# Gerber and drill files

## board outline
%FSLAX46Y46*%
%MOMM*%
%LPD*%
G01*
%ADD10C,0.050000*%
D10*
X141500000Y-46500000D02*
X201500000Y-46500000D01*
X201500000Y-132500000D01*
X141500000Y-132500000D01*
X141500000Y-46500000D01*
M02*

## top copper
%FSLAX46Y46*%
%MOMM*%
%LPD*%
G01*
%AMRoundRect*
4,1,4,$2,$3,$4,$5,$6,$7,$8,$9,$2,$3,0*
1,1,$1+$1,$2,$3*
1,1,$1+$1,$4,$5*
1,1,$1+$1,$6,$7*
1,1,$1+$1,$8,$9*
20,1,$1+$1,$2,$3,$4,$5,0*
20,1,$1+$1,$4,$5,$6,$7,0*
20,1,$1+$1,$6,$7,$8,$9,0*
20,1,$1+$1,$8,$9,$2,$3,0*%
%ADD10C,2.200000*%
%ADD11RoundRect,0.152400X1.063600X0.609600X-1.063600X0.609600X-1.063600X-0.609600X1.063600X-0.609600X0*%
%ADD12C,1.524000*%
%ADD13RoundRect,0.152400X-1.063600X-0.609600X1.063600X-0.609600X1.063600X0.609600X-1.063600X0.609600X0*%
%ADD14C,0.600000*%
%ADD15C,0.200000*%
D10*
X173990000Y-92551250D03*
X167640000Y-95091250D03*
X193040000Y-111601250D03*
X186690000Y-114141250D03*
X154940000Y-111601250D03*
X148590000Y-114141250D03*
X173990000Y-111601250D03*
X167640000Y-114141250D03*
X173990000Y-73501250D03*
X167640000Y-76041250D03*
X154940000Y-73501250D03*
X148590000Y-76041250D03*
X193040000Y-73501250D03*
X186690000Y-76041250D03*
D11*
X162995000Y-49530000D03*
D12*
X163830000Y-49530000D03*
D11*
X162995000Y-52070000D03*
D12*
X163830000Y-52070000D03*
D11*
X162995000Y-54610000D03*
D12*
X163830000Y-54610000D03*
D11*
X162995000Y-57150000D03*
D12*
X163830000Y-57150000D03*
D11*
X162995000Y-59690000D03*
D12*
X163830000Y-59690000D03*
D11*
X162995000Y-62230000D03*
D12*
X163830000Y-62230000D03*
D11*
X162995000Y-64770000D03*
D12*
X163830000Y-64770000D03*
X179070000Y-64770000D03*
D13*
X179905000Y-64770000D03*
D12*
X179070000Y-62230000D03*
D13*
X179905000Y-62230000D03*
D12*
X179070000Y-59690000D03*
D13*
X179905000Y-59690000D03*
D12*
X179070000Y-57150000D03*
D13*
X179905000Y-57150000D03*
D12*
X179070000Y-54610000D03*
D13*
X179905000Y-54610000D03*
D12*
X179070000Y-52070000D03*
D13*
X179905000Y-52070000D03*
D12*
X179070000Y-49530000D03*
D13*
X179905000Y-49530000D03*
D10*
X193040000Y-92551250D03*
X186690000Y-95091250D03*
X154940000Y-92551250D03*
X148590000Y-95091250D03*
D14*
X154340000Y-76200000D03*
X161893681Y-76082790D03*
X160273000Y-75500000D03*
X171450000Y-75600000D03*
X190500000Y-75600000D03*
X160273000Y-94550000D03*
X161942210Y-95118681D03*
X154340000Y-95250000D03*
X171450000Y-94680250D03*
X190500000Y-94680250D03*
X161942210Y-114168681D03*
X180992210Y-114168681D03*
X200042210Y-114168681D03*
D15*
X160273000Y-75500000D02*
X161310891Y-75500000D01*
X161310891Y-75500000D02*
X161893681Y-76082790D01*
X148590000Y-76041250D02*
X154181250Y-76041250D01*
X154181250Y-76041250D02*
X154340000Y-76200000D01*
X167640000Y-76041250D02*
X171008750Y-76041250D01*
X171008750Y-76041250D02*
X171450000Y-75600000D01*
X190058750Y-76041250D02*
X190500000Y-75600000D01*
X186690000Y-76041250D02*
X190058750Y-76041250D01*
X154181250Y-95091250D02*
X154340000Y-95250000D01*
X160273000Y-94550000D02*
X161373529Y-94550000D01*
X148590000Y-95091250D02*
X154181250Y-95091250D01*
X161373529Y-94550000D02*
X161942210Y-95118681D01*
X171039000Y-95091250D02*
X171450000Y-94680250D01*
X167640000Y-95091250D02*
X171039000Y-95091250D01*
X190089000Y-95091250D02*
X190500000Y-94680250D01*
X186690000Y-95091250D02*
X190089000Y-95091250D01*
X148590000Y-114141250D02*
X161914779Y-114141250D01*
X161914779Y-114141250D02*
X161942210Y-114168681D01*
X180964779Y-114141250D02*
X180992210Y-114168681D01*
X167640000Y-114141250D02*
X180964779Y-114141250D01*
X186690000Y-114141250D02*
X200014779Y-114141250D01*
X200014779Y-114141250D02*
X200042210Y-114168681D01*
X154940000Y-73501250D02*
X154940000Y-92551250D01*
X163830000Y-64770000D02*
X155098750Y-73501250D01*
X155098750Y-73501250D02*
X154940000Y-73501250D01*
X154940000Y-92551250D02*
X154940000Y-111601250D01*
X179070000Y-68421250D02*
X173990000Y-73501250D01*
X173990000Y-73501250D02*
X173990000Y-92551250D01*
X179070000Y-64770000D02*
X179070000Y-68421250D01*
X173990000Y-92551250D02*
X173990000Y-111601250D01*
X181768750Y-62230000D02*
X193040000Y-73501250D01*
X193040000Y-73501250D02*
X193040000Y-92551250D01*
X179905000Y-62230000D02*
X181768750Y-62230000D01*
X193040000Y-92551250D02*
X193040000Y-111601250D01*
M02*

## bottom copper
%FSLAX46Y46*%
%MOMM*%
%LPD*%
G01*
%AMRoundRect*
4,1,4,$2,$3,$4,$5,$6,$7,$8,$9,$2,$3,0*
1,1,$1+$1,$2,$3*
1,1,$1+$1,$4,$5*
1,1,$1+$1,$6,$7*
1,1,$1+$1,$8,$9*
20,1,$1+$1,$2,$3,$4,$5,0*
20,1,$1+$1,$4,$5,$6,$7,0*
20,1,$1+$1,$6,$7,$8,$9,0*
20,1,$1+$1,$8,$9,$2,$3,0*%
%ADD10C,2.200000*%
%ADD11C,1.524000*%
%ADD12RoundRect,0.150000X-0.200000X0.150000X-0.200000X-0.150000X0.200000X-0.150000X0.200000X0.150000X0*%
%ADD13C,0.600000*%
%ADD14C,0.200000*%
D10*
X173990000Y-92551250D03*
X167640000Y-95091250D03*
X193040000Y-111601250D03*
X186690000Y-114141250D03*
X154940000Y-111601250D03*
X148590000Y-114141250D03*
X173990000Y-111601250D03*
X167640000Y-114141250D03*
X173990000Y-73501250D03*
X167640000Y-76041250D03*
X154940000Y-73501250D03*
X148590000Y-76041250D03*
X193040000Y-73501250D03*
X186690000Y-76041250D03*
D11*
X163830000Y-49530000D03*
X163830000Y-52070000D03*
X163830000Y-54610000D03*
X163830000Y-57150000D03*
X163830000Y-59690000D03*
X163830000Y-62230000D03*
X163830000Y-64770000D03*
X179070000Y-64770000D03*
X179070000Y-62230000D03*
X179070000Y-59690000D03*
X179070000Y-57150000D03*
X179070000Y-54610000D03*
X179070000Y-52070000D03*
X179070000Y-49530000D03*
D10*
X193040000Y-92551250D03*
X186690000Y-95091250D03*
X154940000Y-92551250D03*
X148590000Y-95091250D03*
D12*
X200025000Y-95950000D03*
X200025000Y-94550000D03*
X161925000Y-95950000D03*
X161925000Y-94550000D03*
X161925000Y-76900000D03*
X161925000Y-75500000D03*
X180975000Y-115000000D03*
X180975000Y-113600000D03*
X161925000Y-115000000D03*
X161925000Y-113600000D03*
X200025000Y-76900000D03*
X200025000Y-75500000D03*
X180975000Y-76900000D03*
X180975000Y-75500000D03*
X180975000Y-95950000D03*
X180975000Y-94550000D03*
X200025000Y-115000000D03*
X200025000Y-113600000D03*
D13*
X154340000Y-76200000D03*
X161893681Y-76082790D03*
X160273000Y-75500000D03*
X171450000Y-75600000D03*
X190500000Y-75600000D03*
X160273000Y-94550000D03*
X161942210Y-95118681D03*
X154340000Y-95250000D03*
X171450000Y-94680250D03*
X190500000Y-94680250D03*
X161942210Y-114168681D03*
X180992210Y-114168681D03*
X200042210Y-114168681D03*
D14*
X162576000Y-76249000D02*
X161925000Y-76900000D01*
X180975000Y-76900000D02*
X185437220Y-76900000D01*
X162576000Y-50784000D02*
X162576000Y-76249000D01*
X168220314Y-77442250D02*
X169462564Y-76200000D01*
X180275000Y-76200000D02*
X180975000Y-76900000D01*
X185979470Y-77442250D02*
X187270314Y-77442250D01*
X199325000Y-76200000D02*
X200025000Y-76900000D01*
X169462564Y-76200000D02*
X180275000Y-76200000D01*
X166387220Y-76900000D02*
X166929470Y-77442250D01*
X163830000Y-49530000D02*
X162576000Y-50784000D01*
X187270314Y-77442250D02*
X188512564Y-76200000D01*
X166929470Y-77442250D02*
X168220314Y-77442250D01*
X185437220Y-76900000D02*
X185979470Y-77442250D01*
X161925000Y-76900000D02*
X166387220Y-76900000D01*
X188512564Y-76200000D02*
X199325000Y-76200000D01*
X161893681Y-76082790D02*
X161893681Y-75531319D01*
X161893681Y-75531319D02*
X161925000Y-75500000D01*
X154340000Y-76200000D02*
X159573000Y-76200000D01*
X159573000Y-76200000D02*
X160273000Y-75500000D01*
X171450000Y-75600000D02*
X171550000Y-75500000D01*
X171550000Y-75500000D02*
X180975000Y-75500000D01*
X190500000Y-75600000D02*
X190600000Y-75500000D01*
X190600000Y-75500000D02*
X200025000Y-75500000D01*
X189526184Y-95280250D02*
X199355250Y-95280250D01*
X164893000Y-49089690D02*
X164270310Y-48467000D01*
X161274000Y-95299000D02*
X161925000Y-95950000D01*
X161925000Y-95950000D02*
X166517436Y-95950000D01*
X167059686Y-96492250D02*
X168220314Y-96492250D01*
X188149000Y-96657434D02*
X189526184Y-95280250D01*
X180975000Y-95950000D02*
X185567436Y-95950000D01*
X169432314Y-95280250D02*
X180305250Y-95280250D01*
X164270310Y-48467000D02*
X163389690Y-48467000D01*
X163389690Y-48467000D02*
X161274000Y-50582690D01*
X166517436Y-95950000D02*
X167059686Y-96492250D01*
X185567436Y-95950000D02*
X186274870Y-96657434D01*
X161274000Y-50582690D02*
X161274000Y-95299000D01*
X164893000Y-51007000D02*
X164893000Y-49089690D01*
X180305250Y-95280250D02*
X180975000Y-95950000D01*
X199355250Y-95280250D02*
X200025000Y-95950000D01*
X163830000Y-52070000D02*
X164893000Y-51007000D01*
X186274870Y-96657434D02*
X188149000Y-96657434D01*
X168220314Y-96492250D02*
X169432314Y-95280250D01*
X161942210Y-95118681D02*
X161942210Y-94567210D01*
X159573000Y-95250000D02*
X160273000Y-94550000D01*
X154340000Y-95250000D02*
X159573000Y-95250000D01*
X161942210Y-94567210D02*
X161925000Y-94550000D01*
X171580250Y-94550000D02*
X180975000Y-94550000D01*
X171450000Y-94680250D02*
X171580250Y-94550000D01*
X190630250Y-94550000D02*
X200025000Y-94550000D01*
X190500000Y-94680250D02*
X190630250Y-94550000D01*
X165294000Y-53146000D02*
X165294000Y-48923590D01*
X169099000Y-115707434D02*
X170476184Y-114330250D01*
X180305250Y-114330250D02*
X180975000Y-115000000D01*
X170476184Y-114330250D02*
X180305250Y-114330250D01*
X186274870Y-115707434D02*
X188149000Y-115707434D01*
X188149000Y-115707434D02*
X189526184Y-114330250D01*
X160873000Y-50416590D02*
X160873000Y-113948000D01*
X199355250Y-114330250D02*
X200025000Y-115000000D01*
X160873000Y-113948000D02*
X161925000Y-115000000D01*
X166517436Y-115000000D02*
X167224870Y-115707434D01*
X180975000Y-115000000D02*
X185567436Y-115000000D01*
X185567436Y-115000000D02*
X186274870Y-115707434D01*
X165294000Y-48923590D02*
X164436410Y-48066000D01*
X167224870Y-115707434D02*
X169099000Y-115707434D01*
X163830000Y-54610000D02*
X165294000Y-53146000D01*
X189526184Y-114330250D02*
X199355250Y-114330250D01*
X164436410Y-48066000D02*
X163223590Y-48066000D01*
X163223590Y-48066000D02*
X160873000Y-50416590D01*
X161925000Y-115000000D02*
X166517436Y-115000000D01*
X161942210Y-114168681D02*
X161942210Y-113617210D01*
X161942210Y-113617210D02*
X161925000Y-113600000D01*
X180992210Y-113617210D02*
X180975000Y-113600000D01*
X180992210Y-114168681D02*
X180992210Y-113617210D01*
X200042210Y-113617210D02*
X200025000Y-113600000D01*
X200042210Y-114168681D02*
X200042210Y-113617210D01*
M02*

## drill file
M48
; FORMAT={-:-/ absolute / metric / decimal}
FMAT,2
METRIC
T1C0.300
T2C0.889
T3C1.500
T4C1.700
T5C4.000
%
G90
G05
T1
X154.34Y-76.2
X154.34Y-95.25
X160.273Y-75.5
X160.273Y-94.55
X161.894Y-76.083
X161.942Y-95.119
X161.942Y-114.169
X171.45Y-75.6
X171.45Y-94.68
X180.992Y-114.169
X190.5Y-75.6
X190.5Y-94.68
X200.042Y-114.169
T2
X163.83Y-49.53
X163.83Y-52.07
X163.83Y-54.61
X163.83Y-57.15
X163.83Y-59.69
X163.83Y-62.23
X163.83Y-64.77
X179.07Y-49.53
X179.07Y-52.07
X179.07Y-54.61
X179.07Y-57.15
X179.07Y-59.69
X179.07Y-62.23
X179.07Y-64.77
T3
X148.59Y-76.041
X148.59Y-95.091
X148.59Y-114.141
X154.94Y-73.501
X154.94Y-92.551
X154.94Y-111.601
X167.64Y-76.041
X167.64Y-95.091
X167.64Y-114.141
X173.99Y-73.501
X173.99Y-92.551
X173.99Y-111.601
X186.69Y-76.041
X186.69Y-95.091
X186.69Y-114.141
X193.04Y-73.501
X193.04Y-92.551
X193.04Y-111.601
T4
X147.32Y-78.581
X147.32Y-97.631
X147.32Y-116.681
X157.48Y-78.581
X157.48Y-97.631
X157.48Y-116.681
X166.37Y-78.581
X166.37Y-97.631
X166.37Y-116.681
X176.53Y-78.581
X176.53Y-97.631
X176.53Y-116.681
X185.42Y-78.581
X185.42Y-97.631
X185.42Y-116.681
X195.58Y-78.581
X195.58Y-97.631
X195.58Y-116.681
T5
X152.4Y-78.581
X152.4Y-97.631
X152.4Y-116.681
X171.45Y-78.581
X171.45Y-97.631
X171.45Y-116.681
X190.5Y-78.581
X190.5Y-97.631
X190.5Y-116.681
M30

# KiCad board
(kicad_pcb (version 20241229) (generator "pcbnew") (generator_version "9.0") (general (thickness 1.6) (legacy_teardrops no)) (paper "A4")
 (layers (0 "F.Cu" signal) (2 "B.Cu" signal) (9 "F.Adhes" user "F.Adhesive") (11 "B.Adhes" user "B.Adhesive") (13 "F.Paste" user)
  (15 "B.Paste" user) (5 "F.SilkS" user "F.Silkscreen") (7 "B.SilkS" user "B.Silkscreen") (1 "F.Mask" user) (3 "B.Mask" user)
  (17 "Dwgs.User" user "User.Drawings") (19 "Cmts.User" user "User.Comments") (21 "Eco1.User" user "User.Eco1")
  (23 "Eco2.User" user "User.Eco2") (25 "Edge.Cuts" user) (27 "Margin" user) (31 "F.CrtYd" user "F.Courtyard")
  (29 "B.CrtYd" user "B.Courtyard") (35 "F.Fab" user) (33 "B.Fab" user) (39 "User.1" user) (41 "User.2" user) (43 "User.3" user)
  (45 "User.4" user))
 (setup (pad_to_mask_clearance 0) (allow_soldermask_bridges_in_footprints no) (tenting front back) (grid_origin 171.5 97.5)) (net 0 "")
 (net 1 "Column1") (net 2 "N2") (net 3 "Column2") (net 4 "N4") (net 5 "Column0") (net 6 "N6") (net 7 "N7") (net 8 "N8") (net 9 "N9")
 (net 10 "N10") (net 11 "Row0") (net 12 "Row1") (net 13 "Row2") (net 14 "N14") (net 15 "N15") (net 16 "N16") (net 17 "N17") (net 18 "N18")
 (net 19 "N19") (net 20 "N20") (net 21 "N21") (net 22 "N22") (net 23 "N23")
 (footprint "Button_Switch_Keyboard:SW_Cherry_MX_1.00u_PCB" (layer "F.Cu") (at 173.99 92.55125)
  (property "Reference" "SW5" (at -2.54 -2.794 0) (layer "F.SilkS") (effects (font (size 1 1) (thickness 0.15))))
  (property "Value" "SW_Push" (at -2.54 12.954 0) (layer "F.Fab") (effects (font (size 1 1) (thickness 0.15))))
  (pad "" np_thru_hole circle (at -7.62 5.08) (size 1.7 1.7) (drill 1.7) (layers "*.Cu" "*.Mask"))
  (pad "" np_thru_hole circle (at -2.54 5.08) (size 4 4) (drill 4) (layers "*.Cu" "*.Mask"))
  (pad "" np_thru_hole circle (at 2.54 5.08) (size 1.7 1.7) (drill 1.7) (layers "*.Cu" "*.Mask"))
  (pad "1" thru_hole circle (at 0 0) (size 2.2 2.2) (drill 1.5) (layers "*.Cu" "*.Mask") (remove_unused_layers no) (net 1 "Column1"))
  (pad "2" thru_hole circle (at -6.35 2.54) (size 2.2 2.2) (drill 1.5) (layers "*.Cu" "*.Mask") (remove_unused_layers no) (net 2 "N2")))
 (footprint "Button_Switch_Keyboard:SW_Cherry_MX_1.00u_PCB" (layer "F.Cu") (at 193.04 111.60125)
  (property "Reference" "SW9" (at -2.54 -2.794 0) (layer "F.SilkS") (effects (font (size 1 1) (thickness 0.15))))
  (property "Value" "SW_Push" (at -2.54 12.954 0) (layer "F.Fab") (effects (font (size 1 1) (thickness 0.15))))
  (pad "" np_thru_hole circle (at -7.62 5.08) (size 1.7 1.7) (drill 1.7) (layers "*.Cu" "*.Mask"))
  (pad "" np_thru_hole circle (at -2.54 5.08) (size 4 4) (drill 4) (layers "*.Cu" "*.Mask"))
  (pad "" np_thru_hole circle (at 2.54 5.08) (size 1.7 1.7) (drill 1.7) (layers "*.Cu" "*.Mask"))
  (pad "1" thru_hole circle (at 0 0) (size 2.2 2.2) (drill 1.5) (layers "*.Cu" "*.Mask") (remove_unused_layers no) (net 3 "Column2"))
  (pad "2" thru_hole circle (at -6.35 2.54) (size 2.2 2.2) (drill 1.5) (layers "*.Cu" "*.Mask") (remove_unused_layers no) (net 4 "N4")))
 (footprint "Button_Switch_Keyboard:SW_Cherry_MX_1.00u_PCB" (layer "F.Cu") (at 154.94 111.60125)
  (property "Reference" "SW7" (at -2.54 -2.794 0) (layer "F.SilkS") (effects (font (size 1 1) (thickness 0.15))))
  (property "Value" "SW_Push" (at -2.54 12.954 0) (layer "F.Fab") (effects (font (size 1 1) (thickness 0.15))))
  (pad "" np_thru_hole circle (at -7.62 5.08) (size 1.7 1.7) (drill 1.7) (layers "*.Cu" "*.Mask"))
  (pad "" np_thru_hole circle (at -2.54 5.08) (size 4 4) (drill 4) (layers "*.Cu" "*.Mask"))
  (pad "" np_thru_hole circle (at 2.54 5.08) (size 1.7 1.7) (drill 1.7) (layers "*.Cu" "*.Mask"))
  (pad "1" thru_hole circle (at 0 0) (size 2.2 2.2) (drill 1.5) (layers "*.Cu" "*.Mask") (remove_unused_layers no) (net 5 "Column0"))
  (pad "2" thru_hole circle (at -6.35 2.54) (size 2.2 2.2) (drill 1.5) (layers "*.Cu" "*.Mask") (remove_unused_layers no) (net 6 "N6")))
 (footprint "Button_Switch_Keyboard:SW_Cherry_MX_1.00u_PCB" (layer "F.Cu") (at 173.99 111.60125)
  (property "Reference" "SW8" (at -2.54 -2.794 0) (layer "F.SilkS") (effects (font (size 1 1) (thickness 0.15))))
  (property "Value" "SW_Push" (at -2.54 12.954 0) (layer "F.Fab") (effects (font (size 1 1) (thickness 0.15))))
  (pad "" np_thru_hole circle (at -7.62 5.08) (size 1.7 1.7) (drill 1.7) (layers "*.Cu" "*.Mask"))
  (pad "" np_thru_hole circle (at -2.54 5.08) (size 4 4) (drill 4) (layers "*.Cu" "*.Mask"))
  (pad "" np_thru_hole circle (at 2.54 5.08) (size 1.7 1.7) (drill 1.7) (layers "*.Cu" "*.Mask"))
  (pad "1" thru_hole circle (at 0 0) (size 2.2 2.2) (drill 1.5) (layers "*.Cu" "*.Mask") (remove_unused_layers no) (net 1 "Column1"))
  (pad "2" thru_hole circle (at -6.35 2.54) (size 2.2 2.2) (drill 1.5) (layers "*.Cu" "*.Mask") (remove_unused_layers no) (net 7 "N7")))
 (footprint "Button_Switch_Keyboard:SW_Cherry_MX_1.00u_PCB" (layer "F.Cu") (at 173.99 73.50125)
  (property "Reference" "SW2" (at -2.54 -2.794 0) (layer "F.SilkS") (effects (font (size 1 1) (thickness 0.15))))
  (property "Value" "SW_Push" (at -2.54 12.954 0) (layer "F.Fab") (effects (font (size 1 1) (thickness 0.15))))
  (pad "" np_thru_hole circle (at -7.62 5.08) (size 1.7 1.7) (drill 1.7) (layers "*.Cu" "*.Mask"))
  (pad "" np_thru_hole circle (at -2.54 5.08) (size 4 4) (drill 4) (layers "*.Cu" "*.Mask"))
  (pad "" np_thru_hole circle (at 2.54 5.08) (size 1.7 1.7) (drill 1.7) (layers "*.Cu" "*.Mask"))
  (pad "1" thru_hole circle (at 0 0) (size 2.2 2.2) (drill 1.5) (layers "*.Cu" "*.Mask") (remove_unused_layers no) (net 1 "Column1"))
  (pad "2" thru_hole circle (at -6.35 2.54) (size 2.2 2.2) (drill 1.5) (layers "*.Cu" "*.Mask") (remove_unused_layers no) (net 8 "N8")))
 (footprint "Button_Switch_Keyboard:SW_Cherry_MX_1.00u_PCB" (layer "F.Cu") (at 154.94 73.50125)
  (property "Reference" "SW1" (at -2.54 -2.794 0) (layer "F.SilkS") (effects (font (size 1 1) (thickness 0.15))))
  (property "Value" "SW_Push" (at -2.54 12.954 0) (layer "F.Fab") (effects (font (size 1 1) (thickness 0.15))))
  (pad "" np_thru_hole circle (at -7.62 5.08) (size 1.7 1.7) (drill 1.7) (layers "*.Cu" "*.Mask"))
  (pad "" np_thru_hole circle (at -2.54 5.08) (size 4 4) (drill 4) (layers "*.Cu" "*.Mask"))
  (pad "" np_thru_hole circle (at 2.54 5.08) (size 1.7 1.7) (drill 1.7) (layers "*.Cu" "*.Mask"))
  (pad "1" thru_hole circle (at 0 0) (size 2.2 2.2) (drill 1.5) (layers "*.Cu" "*.Mask") (remove_unused_layers no) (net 5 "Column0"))
  (pad "2" thru_hole circle (at -6.35 2.54) (size 2.2 2.2) (drill 1.5) (layers "*.Cu" "*.Mask") (remove_unused_layers no) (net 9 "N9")))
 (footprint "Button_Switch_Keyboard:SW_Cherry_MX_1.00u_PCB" (layer "F.Cu") (at 193.04 73.50125)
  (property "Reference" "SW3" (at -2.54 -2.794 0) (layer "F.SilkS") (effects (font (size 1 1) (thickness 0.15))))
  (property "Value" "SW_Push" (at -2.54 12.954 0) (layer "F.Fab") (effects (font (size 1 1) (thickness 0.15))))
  (pad "" np_thru_hole circle (at -7.62 5.08) (size 1.7 1.7) (drill 1.7) (layers "*.Cu" "*.Mask"))
  (pad "" np_thru_hole circle (at -2.54 5.08) (size 4 4) (drill 4) (layers "*.Cu" "*.Mask"))
  (pad "" np_thru_hole circle (at 2.54 5.08) (size 1.7 1.7) (drill 1.7) (layers "*.Cu" "*.Mask"))
  (pad "1" thru_hole circle (at 0 0) (size 2.2 2.2) (drill 1.5) (layers "*.Cu" "*.Mask") (remove_unused_layers no) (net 3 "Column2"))
  (pad "2" thru_hole circle (at -6.35 2.54) (size 2.2 2.2) (drill 1.5) (layers "*.Cu" "*.Mask") (remove_unused_layers no) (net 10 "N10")))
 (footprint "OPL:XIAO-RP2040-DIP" (layer "F.Cu") (at 171.45 57.15)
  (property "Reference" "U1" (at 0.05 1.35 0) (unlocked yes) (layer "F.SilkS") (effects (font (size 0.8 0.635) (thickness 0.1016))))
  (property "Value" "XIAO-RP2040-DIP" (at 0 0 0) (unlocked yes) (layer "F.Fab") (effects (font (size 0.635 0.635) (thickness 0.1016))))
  (pad "1" smd roundrect (at -8.455 -7.62 180) (size 2.432 1.524) (layers "F.Cu" "F.Mask") (roundrect_rratio 0.1) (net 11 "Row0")
   (thermal_bridge_angle 45))
  (pad "1" thru_hole circle (at -7.62 -7.62 180) (size 1.524 1.524) (drill 0.889) (layers "*.Cu" "*.Mask") (remove_unused_layers no)
   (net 11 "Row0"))
  (pad "2" smd roundrect (at -8.455 -5.08 180) (size 2.432 1.524) (layers "F.Cu" "F.Mask") (roundrect_rratio 0.1) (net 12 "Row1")
   (thermal_bridge_angle 45))
  (pad "2" thru_hole circle (at -7.62 -5.08 180) (size 1.524 1.524) (drill 0.889) (layers "*.Cu" "*.Mask") (remove_unused_layers no)
   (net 12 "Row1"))
  (pad "3" smd roundrect (at -8.455 -2.54 180) (size 2.432 1.524) (layers "F.Cu" "F.Mask") (roundrect_rratio 0.1) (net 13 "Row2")
   (thermal_bridge_angle 45))
  (pad "3" thru_hole circle (at -7.62 -2.54 180) (size 1.524 1.524) (drill 0.889) (layers "*.Cu" "*.Mask") (remove_unused_layers no)
   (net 13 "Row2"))
  (pad "4" smd roundrect (at -8.455 0 180) (size 2.432 1.524) (layers "F.Cu" "F.Mask") (roundrect_rratio 0.1) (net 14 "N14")
   (thermal_bridge_angle 45))
  (pad "4" thru_hole circle (at -7.62 0 180) (size 1.524 1.524) (drill 0.889) (layers "*.Cu" "*.Mask") (remove_unused_layers no)
   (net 14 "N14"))
  (pad "5" smd roundrect (at -8.455 2.54 180) (size 2.432 1.524) (layers "F.Cu" "F.Mask") (roundrect_rratio 0.1) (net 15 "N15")
   (thermal_bridge_angle 45))
  (pad "5" thru_hole circle (at -7.62 2.54 180) (size 1.524 1.524) (drill 0.889) (layers "*.Cu" "*.Mask") (remove_unused_layers no)
   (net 15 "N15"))
  (pad "6" smd roundrect (at -8.455 5.08 180) (size 2.432 1.524) (layers "F.Cu" "F.Mask") (roundrect_rratio 0.1) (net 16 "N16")
   (thermal_bridge_angle 45))
  (pad "6" thru_hole circle (at -7.62 5.08 180) (size 1.524 1.524) (drill 0.889) (layers "*.Cu" "*.Mask") (remove_unused_layers no)
   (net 16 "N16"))
  (pad "7" smd roundrect (at -8.455 7.62 180) (size 2.432 1.524) (layers "F.Cu" "F.Mask") (roundrect_rratio 0.1) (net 5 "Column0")
   (thermal_bridge_angle 45))
  (pad "7" thru_hole circle (at -7.62 7.62 180) (size 1.524 1.524) (drill 0.889) (layers "*.Cu" "*.Mask") (remove_unused_layers no)
   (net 5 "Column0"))
  (pad "8" thru_hole circle (at 7.62 7.62) (size 1.524 1.524) (drill 0.889) (layers "*.Cu" "*.Mask") (remove_unused_layers no)
   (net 1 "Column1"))
  (pad "8" smd roundrect (at 8.455 7.62) (size 2.432 1.524) (layers "F.Cu" "F.Mask") (roundrect_rratio 0.1) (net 1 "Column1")
   (thermal_bridge_angle 45))
  (pad "9" thru_hole circle (at 7.62 5.08) (size 1.524 1.524) (drill 0.889) (layers "*.Cu" "*.Mask") (remove_unused_layers no)
   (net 3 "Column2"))
  (pad "9" smd roundrect (at 8.455 5.08) (size 2.432 1.524) (layers "F.Cu" "F.Mask") (roundrect_rratio 0.1) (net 3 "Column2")
   (thermal_bridge_angle 45))
  (pad "10" thru_hole circle (at 7.62 2.54) (size 1.524 1.524) (drill 0.889) (layers "*.Cu" "*.Mask") (remove_unused_layers no)
   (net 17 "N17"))
  (pad "10" smd roundrect (at 8.455 2.54) (size 2.432 1.524) (layers "F.Cu" "F.Mask") (roundrect_rratio 0.1) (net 17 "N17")
   (thermal_bridge_angle 45))
  (pad "11" thru_hole circle (at 7.62 0) (size 1.524 1.524) (drill 0.889) (layers "*.Cu" "*.Mask") (remove_unused_layers no) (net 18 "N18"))
  (pad "11" smd roundrect (at 8.455 0) (size 2.432 1.524) (layers "F.Cu" "F.Mask") (roundrect_rratio 0.1) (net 18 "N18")
   (thermal_bridge_angle 45))
  (pad "12" thru_hole circle (at 7.62 -2.54) (size 1.524 1.524) (drill 0.889) (layers "*.Cu" "*.Mask") (remove_unused_layers no)
   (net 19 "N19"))
  (pad "12" smd roundrect (at 8.455 -2.54) (size 2.432 1.524) (layers "F.Cu" "F.Mask") (roundrect_rratio 0.1) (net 19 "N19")
   (thermal_bridge_angle 45))
  (pad "13" thru_hole circle (at 7.62 -5.08) (size 1.524 1.524) (drill 0.889) (layers "*.Cu" "*.Mask") (remove_unused_layers no)
   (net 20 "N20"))
  (pad "13" smd roundrect (at 8.455 -5.08) (size 2.432 1.524) (layers "F.Cu" "F.Mask") (roundrect_rratio 0.1) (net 20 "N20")
   (thermal_bridge_angle 45))
  (pad "14" thru_hole circle (at 7.62 -7.62) (size 1.524 1.524) (drill 0.889) (layers "*.Cu" "*.Mask") (remove_unused_layers no)
   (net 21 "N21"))
  (pad "14" smd roundrect (at 8.455 -7.62) (size 2.432 1.524) (layers "F.Cu" "F.Mask") (roundrect_rratio 0.1) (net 21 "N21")
   (thermal_bridge_angle 45)))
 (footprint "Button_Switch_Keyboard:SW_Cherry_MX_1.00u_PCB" (layer "F.Cu") (at 193.04 92.55125)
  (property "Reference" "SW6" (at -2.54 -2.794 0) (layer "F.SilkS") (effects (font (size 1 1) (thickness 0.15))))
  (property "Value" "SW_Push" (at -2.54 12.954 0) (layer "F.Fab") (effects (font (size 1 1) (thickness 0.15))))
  (pad "" np_thru_hole circle (at -7.62 5.08) (size 1.7 1.7) (drill 1.7) (layers "*.Cu" "*.Mask"))
  (pad "" np_thru_hole circle (at -2.54 5.08) (size 4 4) (drill 4) (layers "*.Cu" "*.Mask"))
  (pad "" np_thru_hole circle (at 2.54 5.08) (size 1.7 1.7) (drill 1.7) (layers "*.Cu" "*.Mask"))
  (pad "1" thru_hole circle (at 0 0) (size 2.2 2.2) (drill 1.5) (layers "*.Cu" "*.Mask") (remove_unused_layers no) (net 3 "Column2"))
  (pad "2" thru_hole circle (at -6.35 2.54) (size 2.2 2.2) (drill 1.5) (layers "*.Cu" "*.Mask") (remove_unused_layers no) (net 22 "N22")))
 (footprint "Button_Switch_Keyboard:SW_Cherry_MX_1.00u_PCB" (layer "F.Cu") (at 154.94 92.55125)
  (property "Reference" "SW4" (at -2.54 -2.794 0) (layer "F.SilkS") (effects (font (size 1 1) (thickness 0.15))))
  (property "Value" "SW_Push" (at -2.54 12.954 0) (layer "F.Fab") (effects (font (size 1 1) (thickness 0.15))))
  (pad "" np_thru_hole circle (at -7.62 5.08) (size 1.7 1.7) (drill 1.7) (layers "*.Cu" "*.Mask"))
  (pad "" np_thru_hole circle (at -2.54 5.08) (size 4 4) (drill 4) (layers "*.Cu" "*.Mask"))
  (pad "" np_thru_hole circle (at 2.54 5.08) (size 1.7 1.7) (drill 1.7) (layers "*.Cu" "*.Mask"))
  (pad "1" thru_hole circle (at 0 0) (size 2.2 2.2) (drill 1.5) (layers "*.Cu" "*.Mask") (remove_unused_layers no) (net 5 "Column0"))
  (pad "2" thru_hole circle (at -6.35 2.54) (size 2.2 2.2) (drill 1.5) (layers "*.Cu" "*.Mask") (remove_unused_layers no) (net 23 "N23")))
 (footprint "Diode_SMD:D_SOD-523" (layer "B.Cu") (at 200.025 95.25 90)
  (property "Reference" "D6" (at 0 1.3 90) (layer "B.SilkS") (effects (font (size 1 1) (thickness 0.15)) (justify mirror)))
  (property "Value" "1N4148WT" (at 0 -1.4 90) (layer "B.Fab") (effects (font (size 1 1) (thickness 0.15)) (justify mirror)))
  (pad "1" smd roundrect (at -0.7 0 270) (size 0.6 0.7) (layers "B.Cu" "B.Mask" "B.Paste") (roundrect_rratio 0.25) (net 12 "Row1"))
  (pad "2" smd roundrect (at 0.7 0 270) (size 0.6 0.7) (layers "B.Cu" "B.Mask" "B.Paste") (roundrect_rratio 0.25) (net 22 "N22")))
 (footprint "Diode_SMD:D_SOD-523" (layer "B.Cu") (at 161.925 95.25 90)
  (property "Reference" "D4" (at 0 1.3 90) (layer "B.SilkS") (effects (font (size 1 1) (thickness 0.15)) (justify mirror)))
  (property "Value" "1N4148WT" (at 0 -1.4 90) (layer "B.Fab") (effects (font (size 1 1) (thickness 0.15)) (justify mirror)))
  (pad "1" smd roundrect (at -0.7 0 270) (size 0.6 0.7) (layers "B.Cu" "B.Mask" "B.Paste") (roundrect_rratio 0.25) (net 12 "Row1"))
  (pad "2" smd roundrect (at 0.7 0 270) (size 0.6 0.7) (layers "B.Cu" "B.Mask" "B.Paste") (roundrect_rratio 0.25) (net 23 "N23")))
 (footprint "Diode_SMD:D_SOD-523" (layer "B.Cu") (at 161.925 76.2 90)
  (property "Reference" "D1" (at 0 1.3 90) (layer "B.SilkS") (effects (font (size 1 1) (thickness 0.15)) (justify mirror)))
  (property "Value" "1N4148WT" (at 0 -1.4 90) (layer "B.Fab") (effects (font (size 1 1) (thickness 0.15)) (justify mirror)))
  (pad "1" smd roundrect (at -0.7 0 270) (size 0.6 0.7) (layers "B.Cu" "B.Mask" "B.Paste") (roundrect_rratio 0.25) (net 11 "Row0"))
  (pad "2" smd roundrect (at 0.7 0 270) (size 0.6 0.7) (layers "B.Cu" "B.Mask" "B.Paste") (roundrect_rratio 0.25) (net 9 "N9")))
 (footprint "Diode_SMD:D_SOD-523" (layer "B.Cu") (at 180.975 114.3 90)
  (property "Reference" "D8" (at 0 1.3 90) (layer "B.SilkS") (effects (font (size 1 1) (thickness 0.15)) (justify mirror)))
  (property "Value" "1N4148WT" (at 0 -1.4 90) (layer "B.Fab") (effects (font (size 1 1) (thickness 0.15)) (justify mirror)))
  (pad "1" smd roundrect (at -0.7 0 270) (size 0.6 0.7) (layers "B.Cu" "B.Mask" "B.Paste") (roundrect_rratio 0.25) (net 13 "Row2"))
  (pad "2" smd roundrect (at 0.7 0 270) (size 0.6 0.7) (layers "B.Cu" "B.Mask" "B.Paste") (roundrect_rratio 0.25) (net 7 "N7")))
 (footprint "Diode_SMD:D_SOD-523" (layer "B.Cu") (at 161.925 114.3 90)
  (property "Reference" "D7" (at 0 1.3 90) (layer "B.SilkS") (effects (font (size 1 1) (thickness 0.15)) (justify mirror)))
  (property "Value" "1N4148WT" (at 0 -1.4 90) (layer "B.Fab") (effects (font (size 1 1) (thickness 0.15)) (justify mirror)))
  (pad "1" smd roundrect (at -0.7 0 270) (size 0.6 0.7) (layers "B.Cu" "B.Mask" "B.Paste") (roundrect_rratio 0.25) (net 13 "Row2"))
  (pad "2" smd roundrect (at 0.7 0 270) (size 0.6 0.7) (layers "B.Cu" "B.Mask" "B.Paste") (roundrect_rratio 0.25) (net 6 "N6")))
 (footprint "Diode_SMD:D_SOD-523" (layer "B.Cu") (at 200.025 76.2 90)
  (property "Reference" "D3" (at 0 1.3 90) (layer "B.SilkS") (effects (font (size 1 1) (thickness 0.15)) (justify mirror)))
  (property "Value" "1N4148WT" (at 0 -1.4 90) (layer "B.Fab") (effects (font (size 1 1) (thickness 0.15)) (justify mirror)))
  (pad "1" smd roundrect (at -0.7 0 270) (size 0.6 0.7) (layers "B.Cu" "B.Mask" "B.Paste") (roundrect_rratio 0.25) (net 11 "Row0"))
  (pad "2" smd roundrect (at 0.7 0 270) (size 0.6 0.7) (layers "B.Cu" "B.Mask" "B.Paste") (roundrect_rratio 0.25) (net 10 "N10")))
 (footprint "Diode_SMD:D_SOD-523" (layer "B.Cu") (at 180.975 76.2 90)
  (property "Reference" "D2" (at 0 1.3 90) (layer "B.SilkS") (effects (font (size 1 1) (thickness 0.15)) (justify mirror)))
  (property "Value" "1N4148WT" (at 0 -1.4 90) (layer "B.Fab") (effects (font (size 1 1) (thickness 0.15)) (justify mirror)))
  (pad "1" smd roundrect (at -0.7 0 270) (size 0.6 0.7) (layers "B.Cu" "B.Mask" "B.Paste") (roundrect_rratio 0.25) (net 11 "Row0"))
  (pad "2" smd roundrect (at 0.7 0 270) (size 0.6 0.7) (layers "B.Cu" "B.Mask" "B.Paste") (roundrect_rratio 0.25) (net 8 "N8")))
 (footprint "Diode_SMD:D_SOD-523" (layer "B.Cu") (at 180.975 95.25 90)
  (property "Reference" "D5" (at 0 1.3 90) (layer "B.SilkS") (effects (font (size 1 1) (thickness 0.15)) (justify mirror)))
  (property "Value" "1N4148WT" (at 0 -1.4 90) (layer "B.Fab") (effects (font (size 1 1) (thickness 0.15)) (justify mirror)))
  (pad "1" smd roundrect (at -0.7 0 270) (size 0.6 0.7) (layers "B.Cu" "B.Mask" "B.Paste") (roundrect_rratio 0.25) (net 12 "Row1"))
  (pad "2" smd roundrect (at 0.7 0 270) (size 0.6 0.7) (layers "B.Cu" "B.Mask" "B.Paste") (roundrect_rratio 0.25) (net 2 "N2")))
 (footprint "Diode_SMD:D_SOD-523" (layer "B.Cu") (at 200.025 114.3 90)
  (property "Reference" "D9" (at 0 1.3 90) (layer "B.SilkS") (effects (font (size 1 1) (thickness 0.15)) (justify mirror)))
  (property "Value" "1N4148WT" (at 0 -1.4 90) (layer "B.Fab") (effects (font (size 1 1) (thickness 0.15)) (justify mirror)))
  (pad "1" smd roundrect (at -0.7 0 270) (size 0.6 0.7) (layers "B.Cu" "B.Mask" "B.Paste") (roundrect_rratio 0.25) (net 13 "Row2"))
  (pad "2" smd roundrect (at 0.7 0 270) (size 0.6 0.7) (layers "B.Cu" "B.Mask" "B.Paste") (roundrect_rratio 0.25) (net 4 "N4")))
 (gr_rect (start 141.5 46.5) (end 201.5 132.5) (stroke (width 0.05) (type default)) (fill no) (layer "Edge.Cuts"))
 (segment (start 162.576 76.249) (end 161.925 76.9) (width 0.2) (layer "B.Cu") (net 11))
 (segment (start 180.975 76.9) (end 185.43722 76.9) (width 0.2) (layer "B.Cu") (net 11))
 (segment (start 162.576 50.784) (end 162.576 76.249) (width 0.2) (layer "B.Cu") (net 11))
 (segment (start 168.220314 77.44225) (end 169.462564 76.2) (width 0.2) (layer "B.Cu") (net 11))
 (segment (start 180.275 76.2) (end 180.975 76.9) (width 0.2) (layer "B.Cu") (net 11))
 (segment (start 185.97947 77.44225) (end 187.270314 77.44225) (width 0.2) (layer "B.Cu") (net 11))
 (segment (start 199.325 76.2) (end 200.025 76.9) (width 0.2) (layer "B.Cu") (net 11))
 (segment (start 169.462564 76.2) (end 180.275 76.2) (width 0.2) (layer "B.Cu") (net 11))
 (segment (start 166.38722 76.9) (end 166.92947 77.44225) (width 0.2) (layer "B.Cu") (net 11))
 (segment (start 163.83 49.53) (end 162.576 50.784) (width 0.2) (layer "B.Cu") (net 11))
 (segment (start 187.270314 77.44225) (end 188.512564 76.2) (width 0.2) (layer "B.Cu") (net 11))
 (segment (start 166.92947 77.44225) (end 168.220314 77.44225) (width 0.2) (layer "B.Cu") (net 11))
 (segment (start 185.43722 76.9) (end 185.97947 77.44225) (width 0.2) (layer "B.Cu") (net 11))
 (segment (start 161.925 76.9) (end 166.38722 76.9) (width 0.2) (layer "B.Cu") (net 11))
 (segment (start 188.512564 76.2) (end 199.325 76.2) (width 0.2) (layer "B.Cu") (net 11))
 (segment (start 160.273 75.5) (end 161.310891 75.5) (width 0.2) (layer "F.Cu") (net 9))
 (segment (start 161.310891 75.5) (end 161.893681 76.08279) (width 0.2) (layer "F.Cu") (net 9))
 (segment (start 148.59 76.04125) (end 154.18125 76.04125) (width 0.2) (layer "F.Cu") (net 9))
 (segment (start 154.18125 76.04125) (end 154.34 76.2) (width 0.2) (layer "F.Cu") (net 9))
 (via (at 154.34 76.2) (size 0.6) (drill 0.3) (layers "F.Cu" "B.Cu") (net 9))
 (via (at 161.893681 76.08279) (size 0.6) (drill 0.3) (layers "F.Cu" "B.Cu") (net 9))
 (via (at 160.273 75.5) (size 0.6) (drill 0.3) (layers "F.Cu" "B.Cu") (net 9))
 (segment (start 161.893681 76.08279) (end 161.893681 75.531319) (width 0.2) (layer "B.Cu") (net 9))
 (segment (start 161.893681 75.531319) (end 161.925 75.5) (width 0.2) (layer "B.Cu") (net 9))
 (segment (start 154.34 76.2) (end 159.573 76.2) (width 0.2) (layer "B.Cu") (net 9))
 (segment (start 159.573 76.2) (end 160.273 75.5) (width 0.2) (layer "B.Cu") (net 9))
 (segment (start 167.64 76.04125) (end 171.00875 76.04125) (width 0.2) (layer "F.Cu") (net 8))
 (segment (start 171.00875 76.04125) (end 171.45 75.6) (width 0.2) (layer "F.Cu") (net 8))
 (via (at 171.45 75.6) (size 0.6) (drill 0.3) (layers "F.Cu" "B.Cu") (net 8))
 (segment (start 171.45 75.6) (end 171.55 75.5) (width 0.2) (layer "B.Cu") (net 8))
 (segment (start 171.55 75.5) (end 180.975 75.5) (width 0.2) (layer "B.Cu") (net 8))
 (segment (start 190.05875 76.04125) (end 190.5 75.6) (width 0.2) (layer "F.Cu") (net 10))
 (segment (start 186.69 76.04125) (end 190.05875 76.04125) (width 0.2) (layer "F.Cu") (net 10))
 (via (at 190.5 75.6) (size 0.6) (drill 0.3) (layers "F.Cu" "B.Cu") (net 10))
 (segment (start 190.5 75.6) (end 190.6 75.5) (width 0.2) (layer "B.Cu") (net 10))
 (segment (start 190.6 75.5) (end 200.025 75.5) (width 0.2) (layer "B.Cu") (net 10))
 (segment (start 189.526184 95.28025) (end 199.35525 95.28025) (width 0.2) (layer "B.Cu") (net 12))
 (segment (start 164.893 49.08969) (end 164.27031 48.467) (width 0.2) (layer "B.Cu") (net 12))
 (segment (start 161.274 95.299) (end 161.925 95.95) (width 0.2) (layer "B.Cu") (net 12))
 (segment (start 161.925 95.95) (end 166.517436 95.95) (width 0.2) (layer "B.Cu") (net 12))
 (segment (start 167.059686 96.49225) (end 168.220314 96.49225) (width 0.2) (layer "B.Cu") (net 12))
 (segment (start 188.149 96.657434) (end 189.526184 95.28025) (width 0.2) (layer "B.Cu") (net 12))
 (segment (start 180.975 95.95) (end 185.567436 95.95) (width 0.2) (layer "B.Cu") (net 12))
 (segment (start 169.432314 95.28025) (end 180.30525 95.28025) (width 0.2) (layer "B.Cu") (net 12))
 (segment (start 164.27031 48.467) (end 163.38969 48.467) (width 0.2) (layer "B.Cu") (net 12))
 (segment (start 163.38969 48.467) (end 161.274 50.58269) (width 0.2) (layer "B.Cu") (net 12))
 (segment (start 166.517436 95.95) (end 167.059686 96.49225) (width 0.2) (layer "B.Cu") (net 12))
 (segment (start 185.567436 95.95) (end 186.27487 96.657434) (width 0.2) (layer "B.Cu") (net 12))
 (segment (start 161.274 50.58269) (end 161.274 95.299) (width 0.2) (layer "B.Cu") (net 12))
 (segment (start 164.893 51.007) (end 164.893 49.08969) (width 0.2) (layer "B.Cu") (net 12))
 (segment (start 180.30525 95.28025) (end 180.975 95.95) (width 0.2) (layer "B.Cu") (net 12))
 (segment (start 199.35525 95.28025) (end 200.025 95.95) (width 0.2) (layer "B.Cu") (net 12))
 (segment (start 163.83 52.07) (end 164.893 51.007) (width 0.2) (layer "B.Cu") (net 12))
 (segment (start 186.27487 96.657434) (end 188.149 96.657434) (width 0.2) (layer "B.Cu") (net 12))
 (segment (start 168.220314 96.49225) (end 169.432314 95.28025) (width 0.2) (layer "B.Cu") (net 12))
 (segment (start 154.18125 95.09125) (end 154.34 95.25) (width 0.2) (layer "F.Cu") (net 23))
 (segment (start 160.273 94.55) (end 161.373529 94.55) (width 0.2) (layer "F.Cu") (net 23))
 (segment (start 148.59 95.09125) (end 154.18125 95.09125) (width 0.2) (layer "F.Cu") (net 23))
 (segment (start 161.373529 94.55) (end 161.94221 95.118681) (width 0.2) (layer "F.Cu") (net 23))
 (via (at 160.273 94.55) (size 0.6) (drill 0.3) (layers "F.Cu" "B.Cu") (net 23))
 (via (at 161.94221 95.118681) (size 0.6) (drill 0.3) (layers "F.Cu" "B.Cu") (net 23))
 (via (at 154.34 95.25) (size 0.6) (drill 0.3) (layers "F.Cu" "B.Cu") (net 23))
 (segment (start 161.94221 95.118681) (end 161.94221 94.56721) (width 0.2) (layer "B.Cu") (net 23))
 (segment (start 159.573 95.25) (end 160.273 94.55) (width 0.2) (layer "B.Cu") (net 23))
 (segment (start 154.34 95.25) (end 159.573 95.25) (width 0.2) (layer "B.Cu") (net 23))
 (segment (start 161.94221 94.56721) (end 161.925 94.55) (width 0.2) (layer "B.Cu") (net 23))
 (segment (start 171.039 95.09125) (end 171.45 94.68025) (width 0.2) (layer "F.Cu") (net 2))
 (segment (start 167.64 95.09125) (end 171.039 95.09125) (width 0.2) (layer "F.Cu") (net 2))
 (via (at 171.45 94.68025) (size 0.6) (drill 0.3) (layers "F.Cu" "B.Cu") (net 2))
 (segment (start 171.58025 94.55) (end 180.975 94.55) (width 0.2) (layer "B.Cu") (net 2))
 (segment (start 171.45 94.68025) (end 171.58025 94.55) (width 0.2) (layer "B.Cu") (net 2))
 (segment (start 190.089 95.09125) (end 190.5 94.68025) (width 0.2) (layer "F.Cu") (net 22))
 (segment (start 186.69 95.09125) (end 190.089 95.09125) (width 0.2) (layer "F.Cu") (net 22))
 (via (at 190.5 94.68025) (size 0.6) (drill 0.3) (layers "F.Cu" "B.Cu") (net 22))
 (segment (start 190.63025 94.55) (end 200.025 94.55) (width 0.2) (layer "B.Cu") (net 22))
 (segment (start 190.5 94.68025) (end 190.63025 94.55) (width 0.2) (layer "B.Cu") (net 22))
 (segment (start 165.294 53.146) (end 165.294 48.92359) (width 0.2) (layer "B.Cu") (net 13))
 (segment (start 169.099 115.707434) (end 170.476184 114.33025) (width 0.2) (layer "B.Cu") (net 13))
 (segment (start 180.30525 114.33025) (end 180.975 115) (width 0.2) (layer "B.Cu") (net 13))
 (segment (start 170.476184 114.33025) (end 180.30525 114.33025) (width 0.2) (layer "B.Cu") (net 13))
 (segment (start 186.27487 115.707434) (end 188.149 115.707434) (width 0.2) (layer "B.Cu") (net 13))
 (segment (start 188.149 115.707434) (end 189.526184 114.33025) (width 0.2) (layer "B.Cu") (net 13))
 (segment (start 160.873 50.41659) (end 160.873 113.948) (width 0.2) (layer "B.Cu") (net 13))
 (segment (start 199.35525 114.33025) (end 200.025 115) (width 0.2) (layer "B.Cu") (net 13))
 (segment (start 160.873 113.948) (end 161.925 115) (width 0.2) (layer "B.Cu") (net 13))
 (segment (start 166.517436 115) (end 167.22487 115.707434) (width 0.2) (layer "B.Cu") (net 13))
 (segment (start 180.975 115) (end 185.567436 115) (width 0.2) (layer "B.Cu") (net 13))
 (segment (start 185.567436 115) (end 186.27487 115.707434) (width 0.2) (layer "B.Cu") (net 13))
 (segment (start 165.294 48.92359) (end 164.43641 48.066) (width 0.2) (layer "B.Cu") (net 13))
 (segment (start 167.22487 115.707434) (end 169.099 115.707434) (width 0.2) (layer "B.Cu") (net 13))
 (segment (start 163.83 54.61) (end 165.294 53.146) (width 0.2) (layer "B.Cu") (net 13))
 (segment (start 189.526184 114.33025) (end 199.35525 114.33025) (width 0.2) (layer "B.Cu") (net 13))
 (segment (start 164.43641 48.066) (end 163.22359 48.066) (width 0.2) (layer "B.Cu") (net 13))
 (segment (start 163.22359 48.066) (end 160.873 50.41659) (width 0.2) (layer "B.Cu") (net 13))
 (segment (start 161.925 115) (end 166.517436 115) (width 0.2) (layer "B.Cu") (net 13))
 (segment (start 148.59 114.14125) (end 161.914779 114.14125) (width 0.2) (layer "F.Cu") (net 6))
 (segment (start 161.914779 114.14125) (end 161.94221 114.168681) (width 0.2) (layer "F.Cu") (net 6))
 (via (at 161.94221 114.168681) (size 0.6) (drill 0.3) (layers "F.Cu" "B.Cu") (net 6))
 (segment (start 161.94221 114.168681) (end 161.94221 113.61721) (width 0.2) (layer "B.Cu") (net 6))
 (segment (start 161.94221 113.61721) (end 161.925 113.6) (width 0.2) (layer "B.Cu") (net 6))
 (segment (start 180.964779 114.14125) (end 180.99221 114.168681) (width 0.2) (layer "F.Cu") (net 7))
 (segment (start 167.64 114.14125) (end 180.964779 114.14125) (width 0.2) (layer "F.Cu") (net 7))
 (via (at 180.99221 114.168681) (size 0.6) (drill 0.3) (layers "F.Cu" "B.Cu") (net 7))
 (segment (start 180.99221 113.61721) (end 180.975 113.6) (width 0.2) (layer "B.Cu") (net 7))
 (segment (start 180.99221 114.168681) (end 180.99221 113.61721) (width 0.2) (layer "B.Cu") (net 7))
 (segment (start 186.69 114.14125) (end 200.014779 114.14125) (width 0.2) (layer "F.Cu") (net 4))
 (segment (start 200.014779 114.14125) (end 200.04221 114.168681) (width 0.2) (layer "F.Cu") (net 4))
 (via (at 200.04221 114.168681) (size 0.6) (drill 0.3) (layers "F.Cu" "B.Cu") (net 4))
 (segment (start 200.04221 113.61721) (end 200.025 113.6) (width 0.2) (layer "B.Cu") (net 4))
 (segment (start 200.04221 114.168681) (end 200.04221 113.61721) (width 0.2) (layer "B.Cu") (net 4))
 (segment (start 154.94 73.50125) (end 154.94 92.55125) (width 0.2) (layer "F.Cu") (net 5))
 (segment (start 163.83 64.77) (end 155.09875 73.50125) (width 0.2) (layer "F.Cu") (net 5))
 (segment (start 155.09875 73.50125) (end 154.94 73.50125) (width 0.2) (layer "F.Cu") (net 5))
 (segment (start 154.94 92.55125) (end 154.94 111.60125) (width 0.2) (layer "F.Cu") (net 5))
 (segment (start 179.07 68.42125) (end 173.99 73.50125) (width 0.2) (layer "F.Cu") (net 1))
 (segment (start 173.99 73.50125) (end 173.99 92.55125) (width 0.2) (layer "F.Cu") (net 1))
 (segment (start 179.07 64.77) (end 179.07 68.42125) (width 0.2) (layer "F.Cu") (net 1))
 (segment (start 173.99 92.55125) (end 173.99 111.60125) (width 0.2) (layer "F.Cu") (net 1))
 (segment (start 181.76875 62.23) (end 193.04 73.50125) (width 0.2) (layer "F.Cu") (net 3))
 (segment (start 193.04 73.50125) (end 193.04 92.55125) (width 0.2) (layer "F.Cu") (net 3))
 (segment (start 179.905 62.23) (end 181.76875 62.23) (width 0.2) (layer "F.Cu") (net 3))
 (segment (start 193.04 92.55125) (end 193.04 111.60125) (width 0.2) (layer "F.Cu") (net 3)))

